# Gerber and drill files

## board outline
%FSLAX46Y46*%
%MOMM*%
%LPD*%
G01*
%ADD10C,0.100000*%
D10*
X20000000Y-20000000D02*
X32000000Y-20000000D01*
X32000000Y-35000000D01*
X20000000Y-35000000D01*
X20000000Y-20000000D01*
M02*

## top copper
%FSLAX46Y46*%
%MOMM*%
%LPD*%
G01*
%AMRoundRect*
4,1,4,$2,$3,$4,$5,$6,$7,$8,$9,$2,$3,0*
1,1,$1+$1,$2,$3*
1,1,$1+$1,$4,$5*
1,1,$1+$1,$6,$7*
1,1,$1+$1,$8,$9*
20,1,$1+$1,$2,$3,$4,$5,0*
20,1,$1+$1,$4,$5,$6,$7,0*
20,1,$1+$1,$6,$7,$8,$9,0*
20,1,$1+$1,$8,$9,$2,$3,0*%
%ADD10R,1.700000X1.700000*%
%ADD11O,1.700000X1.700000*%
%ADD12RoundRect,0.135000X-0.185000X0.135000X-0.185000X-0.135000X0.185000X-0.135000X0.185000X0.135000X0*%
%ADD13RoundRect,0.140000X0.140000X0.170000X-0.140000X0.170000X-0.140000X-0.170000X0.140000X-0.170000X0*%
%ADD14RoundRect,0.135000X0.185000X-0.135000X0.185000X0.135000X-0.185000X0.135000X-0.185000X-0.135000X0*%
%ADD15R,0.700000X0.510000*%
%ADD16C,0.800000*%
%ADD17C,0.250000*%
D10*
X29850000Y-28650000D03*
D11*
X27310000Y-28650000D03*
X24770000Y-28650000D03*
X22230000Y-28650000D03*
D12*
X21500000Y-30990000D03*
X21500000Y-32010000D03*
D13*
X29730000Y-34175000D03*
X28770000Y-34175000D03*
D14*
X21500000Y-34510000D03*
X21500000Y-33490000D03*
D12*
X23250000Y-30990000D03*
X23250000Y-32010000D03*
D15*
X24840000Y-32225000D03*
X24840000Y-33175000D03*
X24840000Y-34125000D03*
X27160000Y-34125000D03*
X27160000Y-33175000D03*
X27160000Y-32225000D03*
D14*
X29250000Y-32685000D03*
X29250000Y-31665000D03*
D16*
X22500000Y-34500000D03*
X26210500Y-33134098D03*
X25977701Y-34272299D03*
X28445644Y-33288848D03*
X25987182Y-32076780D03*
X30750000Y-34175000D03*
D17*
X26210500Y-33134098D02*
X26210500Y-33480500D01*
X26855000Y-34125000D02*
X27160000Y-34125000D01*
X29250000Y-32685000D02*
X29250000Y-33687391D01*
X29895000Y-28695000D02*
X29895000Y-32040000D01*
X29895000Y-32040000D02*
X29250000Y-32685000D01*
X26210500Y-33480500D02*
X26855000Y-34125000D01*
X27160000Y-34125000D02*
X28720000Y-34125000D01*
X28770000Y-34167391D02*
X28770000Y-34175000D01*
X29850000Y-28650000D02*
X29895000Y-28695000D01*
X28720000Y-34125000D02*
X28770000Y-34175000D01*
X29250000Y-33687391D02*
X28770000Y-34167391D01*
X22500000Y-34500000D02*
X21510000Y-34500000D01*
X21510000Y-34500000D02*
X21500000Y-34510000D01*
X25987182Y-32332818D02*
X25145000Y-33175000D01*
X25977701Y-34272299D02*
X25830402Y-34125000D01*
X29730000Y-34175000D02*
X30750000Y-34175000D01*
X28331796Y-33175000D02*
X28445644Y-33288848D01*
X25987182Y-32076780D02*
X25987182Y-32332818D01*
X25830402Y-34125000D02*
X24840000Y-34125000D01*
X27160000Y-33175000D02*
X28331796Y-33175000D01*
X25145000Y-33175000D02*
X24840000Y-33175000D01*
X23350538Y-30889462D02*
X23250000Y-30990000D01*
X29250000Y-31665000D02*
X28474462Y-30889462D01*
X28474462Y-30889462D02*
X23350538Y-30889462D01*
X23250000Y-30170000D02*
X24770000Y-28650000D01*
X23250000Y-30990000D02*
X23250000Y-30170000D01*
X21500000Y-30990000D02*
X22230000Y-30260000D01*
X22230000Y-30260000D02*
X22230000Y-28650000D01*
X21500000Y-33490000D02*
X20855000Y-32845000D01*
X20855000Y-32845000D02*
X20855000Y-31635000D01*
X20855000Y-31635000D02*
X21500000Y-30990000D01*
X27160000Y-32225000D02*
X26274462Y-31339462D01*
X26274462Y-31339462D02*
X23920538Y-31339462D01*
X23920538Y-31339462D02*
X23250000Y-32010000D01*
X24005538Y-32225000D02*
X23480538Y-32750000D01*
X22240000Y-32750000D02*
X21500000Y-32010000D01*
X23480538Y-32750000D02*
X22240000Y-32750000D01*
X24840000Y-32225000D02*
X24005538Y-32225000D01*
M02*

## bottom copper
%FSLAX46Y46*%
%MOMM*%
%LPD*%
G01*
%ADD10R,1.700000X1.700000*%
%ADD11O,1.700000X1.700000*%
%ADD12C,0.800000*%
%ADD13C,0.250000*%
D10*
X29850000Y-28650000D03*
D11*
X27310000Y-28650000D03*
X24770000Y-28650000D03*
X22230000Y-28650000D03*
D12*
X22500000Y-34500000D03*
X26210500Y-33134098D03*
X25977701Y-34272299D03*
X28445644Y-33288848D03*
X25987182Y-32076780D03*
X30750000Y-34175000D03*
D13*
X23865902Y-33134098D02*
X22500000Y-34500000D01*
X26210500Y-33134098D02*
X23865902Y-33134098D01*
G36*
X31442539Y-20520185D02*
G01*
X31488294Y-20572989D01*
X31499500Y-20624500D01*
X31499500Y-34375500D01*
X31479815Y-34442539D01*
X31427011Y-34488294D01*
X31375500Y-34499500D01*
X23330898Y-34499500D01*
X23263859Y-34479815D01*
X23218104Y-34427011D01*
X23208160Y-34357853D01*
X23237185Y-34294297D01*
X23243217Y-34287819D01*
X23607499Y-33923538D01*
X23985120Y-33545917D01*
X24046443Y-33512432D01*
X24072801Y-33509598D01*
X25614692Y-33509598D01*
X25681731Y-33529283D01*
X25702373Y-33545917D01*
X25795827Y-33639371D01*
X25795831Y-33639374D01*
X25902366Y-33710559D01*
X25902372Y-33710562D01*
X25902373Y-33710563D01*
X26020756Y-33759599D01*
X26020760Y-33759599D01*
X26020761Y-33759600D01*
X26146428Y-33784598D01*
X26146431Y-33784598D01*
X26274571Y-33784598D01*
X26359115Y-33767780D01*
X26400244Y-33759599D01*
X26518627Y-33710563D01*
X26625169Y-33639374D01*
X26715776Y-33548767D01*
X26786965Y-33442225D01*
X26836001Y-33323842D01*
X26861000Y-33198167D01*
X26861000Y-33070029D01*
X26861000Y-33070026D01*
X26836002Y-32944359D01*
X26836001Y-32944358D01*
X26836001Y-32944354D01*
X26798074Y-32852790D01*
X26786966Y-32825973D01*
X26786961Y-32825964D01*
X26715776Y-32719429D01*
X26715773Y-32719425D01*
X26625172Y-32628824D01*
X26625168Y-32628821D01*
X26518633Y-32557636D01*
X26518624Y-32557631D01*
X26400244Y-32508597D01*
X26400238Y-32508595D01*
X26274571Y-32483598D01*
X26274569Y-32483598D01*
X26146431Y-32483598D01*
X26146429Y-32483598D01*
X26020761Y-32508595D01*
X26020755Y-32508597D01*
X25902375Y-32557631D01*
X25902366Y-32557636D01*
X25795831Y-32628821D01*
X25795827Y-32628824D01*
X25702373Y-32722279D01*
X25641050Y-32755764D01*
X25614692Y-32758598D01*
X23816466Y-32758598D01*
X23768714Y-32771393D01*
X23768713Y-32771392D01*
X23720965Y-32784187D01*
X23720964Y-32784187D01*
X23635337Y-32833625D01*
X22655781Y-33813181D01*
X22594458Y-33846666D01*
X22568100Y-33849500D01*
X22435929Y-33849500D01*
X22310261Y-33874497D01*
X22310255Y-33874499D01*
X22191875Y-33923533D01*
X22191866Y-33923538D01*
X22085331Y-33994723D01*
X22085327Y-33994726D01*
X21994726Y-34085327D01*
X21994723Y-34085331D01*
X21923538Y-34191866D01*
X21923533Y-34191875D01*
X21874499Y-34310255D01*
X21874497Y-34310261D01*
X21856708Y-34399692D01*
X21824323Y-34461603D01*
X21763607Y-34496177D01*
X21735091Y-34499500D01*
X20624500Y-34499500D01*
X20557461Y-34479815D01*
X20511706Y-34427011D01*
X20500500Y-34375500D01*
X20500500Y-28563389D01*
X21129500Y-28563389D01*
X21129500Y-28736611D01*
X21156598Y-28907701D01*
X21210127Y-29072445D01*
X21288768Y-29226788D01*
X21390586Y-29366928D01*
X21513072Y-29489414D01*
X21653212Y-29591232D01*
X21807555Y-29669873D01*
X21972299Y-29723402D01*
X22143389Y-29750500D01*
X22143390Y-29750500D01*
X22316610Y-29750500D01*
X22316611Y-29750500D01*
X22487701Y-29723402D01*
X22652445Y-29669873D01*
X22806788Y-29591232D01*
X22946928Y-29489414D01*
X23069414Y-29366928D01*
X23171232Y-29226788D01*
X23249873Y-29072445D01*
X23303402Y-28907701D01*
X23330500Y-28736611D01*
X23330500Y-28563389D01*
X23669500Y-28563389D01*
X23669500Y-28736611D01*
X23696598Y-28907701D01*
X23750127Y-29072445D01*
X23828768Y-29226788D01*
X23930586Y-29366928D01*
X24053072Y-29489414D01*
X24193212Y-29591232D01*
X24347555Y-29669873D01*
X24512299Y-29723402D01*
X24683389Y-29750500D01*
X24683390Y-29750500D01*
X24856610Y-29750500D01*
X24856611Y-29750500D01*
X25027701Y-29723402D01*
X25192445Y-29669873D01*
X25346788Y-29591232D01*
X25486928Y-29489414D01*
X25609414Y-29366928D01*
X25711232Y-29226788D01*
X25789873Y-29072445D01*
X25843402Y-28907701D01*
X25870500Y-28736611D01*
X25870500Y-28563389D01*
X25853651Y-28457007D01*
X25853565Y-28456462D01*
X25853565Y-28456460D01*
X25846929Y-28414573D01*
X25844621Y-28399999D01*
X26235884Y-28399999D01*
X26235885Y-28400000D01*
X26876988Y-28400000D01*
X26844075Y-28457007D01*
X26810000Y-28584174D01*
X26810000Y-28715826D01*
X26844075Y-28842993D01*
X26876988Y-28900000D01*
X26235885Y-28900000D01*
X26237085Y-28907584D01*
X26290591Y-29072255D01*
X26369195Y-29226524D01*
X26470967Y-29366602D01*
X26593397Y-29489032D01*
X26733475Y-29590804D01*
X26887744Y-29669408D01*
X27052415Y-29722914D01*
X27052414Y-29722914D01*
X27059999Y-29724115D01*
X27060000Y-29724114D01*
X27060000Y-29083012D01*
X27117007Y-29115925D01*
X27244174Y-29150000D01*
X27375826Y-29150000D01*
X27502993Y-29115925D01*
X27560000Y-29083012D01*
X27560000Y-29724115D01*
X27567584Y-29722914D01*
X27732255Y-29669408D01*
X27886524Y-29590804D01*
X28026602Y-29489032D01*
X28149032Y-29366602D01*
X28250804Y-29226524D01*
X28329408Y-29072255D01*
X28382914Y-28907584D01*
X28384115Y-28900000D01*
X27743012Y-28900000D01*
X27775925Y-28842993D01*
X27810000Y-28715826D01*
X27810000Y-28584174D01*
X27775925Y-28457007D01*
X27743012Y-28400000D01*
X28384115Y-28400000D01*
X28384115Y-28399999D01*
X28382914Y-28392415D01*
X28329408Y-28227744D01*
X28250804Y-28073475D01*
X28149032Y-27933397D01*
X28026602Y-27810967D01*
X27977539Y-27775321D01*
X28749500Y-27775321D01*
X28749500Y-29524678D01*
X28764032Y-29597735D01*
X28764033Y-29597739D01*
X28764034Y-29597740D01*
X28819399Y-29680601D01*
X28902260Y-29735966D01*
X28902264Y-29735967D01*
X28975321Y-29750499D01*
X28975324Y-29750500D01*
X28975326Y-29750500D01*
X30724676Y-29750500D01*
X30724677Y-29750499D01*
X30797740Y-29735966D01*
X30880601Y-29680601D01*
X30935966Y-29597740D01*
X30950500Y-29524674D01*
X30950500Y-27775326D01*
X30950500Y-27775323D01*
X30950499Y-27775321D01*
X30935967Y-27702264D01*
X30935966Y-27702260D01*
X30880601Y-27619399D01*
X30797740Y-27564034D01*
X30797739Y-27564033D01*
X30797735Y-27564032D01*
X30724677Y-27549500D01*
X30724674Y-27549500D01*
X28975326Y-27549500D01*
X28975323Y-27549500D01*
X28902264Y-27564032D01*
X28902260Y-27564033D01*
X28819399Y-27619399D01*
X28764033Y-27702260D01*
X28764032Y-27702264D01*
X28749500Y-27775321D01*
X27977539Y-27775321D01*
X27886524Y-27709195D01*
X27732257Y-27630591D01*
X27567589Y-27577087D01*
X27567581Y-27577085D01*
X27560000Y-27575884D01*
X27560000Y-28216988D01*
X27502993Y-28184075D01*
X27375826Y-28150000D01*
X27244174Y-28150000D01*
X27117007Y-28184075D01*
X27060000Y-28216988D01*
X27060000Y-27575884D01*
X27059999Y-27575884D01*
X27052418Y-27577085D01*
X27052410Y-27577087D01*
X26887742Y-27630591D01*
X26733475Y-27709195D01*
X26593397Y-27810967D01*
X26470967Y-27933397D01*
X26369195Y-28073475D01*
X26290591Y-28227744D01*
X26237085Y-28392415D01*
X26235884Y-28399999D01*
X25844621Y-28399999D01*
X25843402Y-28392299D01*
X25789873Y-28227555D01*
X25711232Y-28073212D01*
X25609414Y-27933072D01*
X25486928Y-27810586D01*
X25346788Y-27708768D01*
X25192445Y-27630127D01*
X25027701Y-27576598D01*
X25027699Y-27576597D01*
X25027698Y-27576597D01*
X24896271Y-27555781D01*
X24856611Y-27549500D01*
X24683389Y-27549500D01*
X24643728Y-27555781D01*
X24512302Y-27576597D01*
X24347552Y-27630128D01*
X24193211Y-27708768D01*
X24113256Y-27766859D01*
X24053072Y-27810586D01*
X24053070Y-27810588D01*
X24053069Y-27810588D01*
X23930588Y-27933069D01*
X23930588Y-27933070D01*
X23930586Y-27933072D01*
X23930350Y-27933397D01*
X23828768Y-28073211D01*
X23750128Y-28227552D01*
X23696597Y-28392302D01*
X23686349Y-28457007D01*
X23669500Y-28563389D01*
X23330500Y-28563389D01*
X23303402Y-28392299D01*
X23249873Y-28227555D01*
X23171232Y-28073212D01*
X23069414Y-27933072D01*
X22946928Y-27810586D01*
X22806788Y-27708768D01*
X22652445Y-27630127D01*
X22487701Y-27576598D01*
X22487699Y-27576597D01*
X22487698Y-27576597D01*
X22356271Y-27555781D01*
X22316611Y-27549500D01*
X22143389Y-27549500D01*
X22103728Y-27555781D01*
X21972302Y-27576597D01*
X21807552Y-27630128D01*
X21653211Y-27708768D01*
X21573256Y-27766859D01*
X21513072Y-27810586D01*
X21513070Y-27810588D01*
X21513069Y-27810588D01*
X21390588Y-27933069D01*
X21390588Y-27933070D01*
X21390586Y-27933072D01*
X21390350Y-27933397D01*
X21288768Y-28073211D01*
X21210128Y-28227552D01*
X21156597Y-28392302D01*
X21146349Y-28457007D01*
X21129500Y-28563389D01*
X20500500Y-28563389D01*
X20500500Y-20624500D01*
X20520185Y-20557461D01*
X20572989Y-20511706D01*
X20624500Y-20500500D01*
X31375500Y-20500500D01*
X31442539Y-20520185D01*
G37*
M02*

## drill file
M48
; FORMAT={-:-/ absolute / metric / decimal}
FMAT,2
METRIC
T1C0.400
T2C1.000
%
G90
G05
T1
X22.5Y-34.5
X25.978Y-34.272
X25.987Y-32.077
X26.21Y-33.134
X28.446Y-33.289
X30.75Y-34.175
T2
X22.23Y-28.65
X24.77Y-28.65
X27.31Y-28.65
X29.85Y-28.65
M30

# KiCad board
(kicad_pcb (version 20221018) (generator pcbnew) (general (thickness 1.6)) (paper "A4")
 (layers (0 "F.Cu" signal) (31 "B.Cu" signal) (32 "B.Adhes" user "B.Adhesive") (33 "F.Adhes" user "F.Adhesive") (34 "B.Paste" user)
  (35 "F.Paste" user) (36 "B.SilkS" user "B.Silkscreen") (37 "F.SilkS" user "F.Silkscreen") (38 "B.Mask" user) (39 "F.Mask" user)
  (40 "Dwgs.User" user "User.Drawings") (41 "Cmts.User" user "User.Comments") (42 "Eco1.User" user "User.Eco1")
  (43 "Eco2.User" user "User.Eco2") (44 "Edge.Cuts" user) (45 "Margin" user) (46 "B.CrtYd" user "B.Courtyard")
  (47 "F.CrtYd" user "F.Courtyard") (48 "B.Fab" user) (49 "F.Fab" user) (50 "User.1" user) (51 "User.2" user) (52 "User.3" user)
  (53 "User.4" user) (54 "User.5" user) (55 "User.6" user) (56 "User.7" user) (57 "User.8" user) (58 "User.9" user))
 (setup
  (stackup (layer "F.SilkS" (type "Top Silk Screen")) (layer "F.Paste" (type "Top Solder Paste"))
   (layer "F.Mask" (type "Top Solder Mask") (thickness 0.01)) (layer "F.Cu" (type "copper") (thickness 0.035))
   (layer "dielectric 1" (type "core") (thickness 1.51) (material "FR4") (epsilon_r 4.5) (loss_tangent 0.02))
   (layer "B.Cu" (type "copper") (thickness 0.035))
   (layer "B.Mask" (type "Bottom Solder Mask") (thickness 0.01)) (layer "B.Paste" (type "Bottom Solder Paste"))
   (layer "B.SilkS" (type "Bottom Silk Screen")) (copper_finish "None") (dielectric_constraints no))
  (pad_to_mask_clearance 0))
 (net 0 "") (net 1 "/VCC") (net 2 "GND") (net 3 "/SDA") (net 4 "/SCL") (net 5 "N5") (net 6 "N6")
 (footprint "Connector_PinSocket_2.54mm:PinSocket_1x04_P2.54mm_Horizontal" (layer "F.Cu") (at 29.85 28.65 -90)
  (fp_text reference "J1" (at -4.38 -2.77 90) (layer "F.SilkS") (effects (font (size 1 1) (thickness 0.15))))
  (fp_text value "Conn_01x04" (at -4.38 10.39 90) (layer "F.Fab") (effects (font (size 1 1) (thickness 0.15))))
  (pad "1" thru_hole rect (at 0 0 270) (size 1.7 1.7) (drill 1) (layers "*.Cu" "*.Mask") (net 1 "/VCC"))
  (pad "2" thru_hole oval (at 0 2.54 270) (size 1.7 1.7) (drill 1) (layers "*.Cu" "*.Mask") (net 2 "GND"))
  (pad "3" thru_hole oval (at 0 5.08 270) (size 1.7 1.7) (drill 1) (layers "*.Cu" "*.Mask") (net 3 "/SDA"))
  (pad "4" thru_hole oval (at 0 7.62 270) (size 1.7 1.7) (drill 1) (layers "*.Cu" "*.Mask") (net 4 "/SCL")))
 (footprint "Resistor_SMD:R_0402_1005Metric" (layer "F.Cu") (at 21.5 31.5 -90)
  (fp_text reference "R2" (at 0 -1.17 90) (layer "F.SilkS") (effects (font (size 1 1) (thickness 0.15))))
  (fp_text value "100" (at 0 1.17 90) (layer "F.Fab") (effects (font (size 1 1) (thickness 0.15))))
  (pad "1" smd roundrect (at -0.51 0 270) (size 0.54 0.64) (layers "F.Cu" "F.Paste" "F.Mask") (roundrect_rratio 0.25) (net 4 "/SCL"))
  (pad "2" smd roundrect (at 0.51 0 270) (size 0.54 0.64) (layers "F.Cu" "F.Paste" "F.Mask") (roundrect_rratio 0.25) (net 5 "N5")))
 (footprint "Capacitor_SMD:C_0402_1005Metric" (layer "F.Cu") (at 29.25 34.175 180)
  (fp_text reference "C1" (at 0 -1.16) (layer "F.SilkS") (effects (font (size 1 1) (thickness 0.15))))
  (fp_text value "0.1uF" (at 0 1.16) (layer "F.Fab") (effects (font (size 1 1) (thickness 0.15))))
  (pad "1" smd roundrect (at -0.48 0 180) (size 0.56 0.62) (layers "F.Cu" "F.Paste" "F.Mask") (roundrect_rratio 0.25) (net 2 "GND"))
  (pad "2" smd roundrect (at 0.48 0 180) (size 0.56 0.62) (layers "F.Cu" "F.Paste" "F.Mask") (roundrect_rratio 0.25) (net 1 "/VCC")))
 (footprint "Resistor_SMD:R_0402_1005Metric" (layer "F.Cu") (at 21.5 34 90)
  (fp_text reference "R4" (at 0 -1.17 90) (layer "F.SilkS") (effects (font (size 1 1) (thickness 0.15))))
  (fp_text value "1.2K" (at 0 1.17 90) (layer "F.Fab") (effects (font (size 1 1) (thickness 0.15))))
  (pad "1" smd roundrect (at -0.51 0 90) (size 0.54 0.64) (layers "F.Cu" "F.Paste" "F.Mask") (roundrect_rratio 0.25) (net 1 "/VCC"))
  (pad "2" smd roundrect (at 0.51 0 90) (size 0.54 0.64) (layers "F.Cu" "F.Paste" "F.Mask") (roundrect_rratio 0.25) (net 4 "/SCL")))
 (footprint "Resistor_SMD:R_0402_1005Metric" (layer "F.Cu") (at 23.25 31.5 -90)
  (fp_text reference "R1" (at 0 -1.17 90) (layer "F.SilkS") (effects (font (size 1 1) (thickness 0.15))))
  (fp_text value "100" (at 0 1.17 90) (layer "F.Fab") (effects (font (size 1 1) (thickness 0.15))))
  (pad "1" smd roundrect (at -0.51 0 270) (size 0.54 0.64) (layers "F.Cu" "F.Paste" "F.Mask") (roundrect_rratio 0.25) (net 3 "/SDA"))
  (pad "2" smd roundrect (at 0.51 0 270) (size 0.54 0.64) (layers "F.Cu" "F.Paste" "F.Mask") (roundrect_rratio 0.25) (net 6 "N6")))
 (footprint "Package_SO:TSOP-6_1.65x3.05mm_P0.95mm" (layer "F.Cu") (at 26 33.175)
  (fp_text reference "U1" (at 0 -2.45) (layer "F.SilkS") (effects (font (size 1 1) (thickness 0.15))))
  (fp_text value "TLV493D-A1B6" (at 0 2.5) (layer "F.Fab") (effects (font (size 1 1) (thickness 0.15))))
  (pad "1" smd rect (at -1.16 -0.95) (size 0.7 0.51) (layers "F.Cu" "F.Paste" "F.Mask") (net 5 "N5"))
  (pad "2" smd rect (at -1.16 0) (size 0.7 0.51) (layers "F.Cu" "F.Paste" "F.Mask") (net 2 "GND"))
  (pad "3" smd rect (at -1.16 0.95) (size 0.7 0.51) (layers "F.Cu" "F.Paste" "F.Mask") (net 2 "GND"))
  (pad "4" smd rect (at 1.16 0.95) (size 0.7 0.51) (layers "F.Cu" "F.Paste" "F.Mask") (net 1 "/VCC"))
  (pad "5" smd rect (at 1.16 0) (size 0.7 0.51) (layers "F.Cu" "F.Paste" "F.Mask") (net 2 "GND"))
  (pad "6" smd rect (at 1.16 -0.95) (size 0.7 0.51) (layers "F.Cu" "F.Paste" "F.Mask") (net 6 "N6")))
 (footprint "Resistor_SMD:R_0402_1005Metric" (layer "F.Cu") (at 29.25 32.175 90)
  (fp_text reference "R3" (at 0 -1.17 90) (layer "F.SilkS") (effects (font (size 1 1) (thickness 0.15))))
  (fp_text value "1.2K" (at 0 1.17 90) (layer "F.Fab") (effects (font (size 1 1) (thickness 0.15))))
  (pad "1" smd roundrect (at -0.51 0 90) (size 0.54 0.64) (layers "F.Cu" "F.Paste" "F.Mask") (roundrect_rratio 0.25) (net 1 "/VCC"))
  (pad "2" smd roundrect (at 0.51 0 90) (size 0.54 0.64) (layers "F.Cu" "F.Paste" "F.Mask") (roundrect_rratio 0.25) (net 3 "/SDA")))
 (gr_rect (start 20 20) (end 32 35) (stroke (width 0.1) (type default)) (fill none) (layer "Edge.Cuts"))
 (segment (start 26.2105 33.134098) (end 26.2105 33.4805) (width 0.25) (layer "F.Cu") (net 1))
 (segment (start 26.855 34.125) (end 27.16 34.125) (width 0.25) (layer "F.Cu") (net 1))
 (segment (start 29.25 32.685) (end 29.25 33.687391) (width 0.25) (layer "F.Cu") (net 1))
 (segment (start 29.895 28.695) (end 29.895 32.04) (width 0.25) (layer "F.Cu") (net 1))
 (segment (start 29.895 32.04) (end 29.25 32.685) (width 0.25) (layer "F.Cu") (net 1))
 (segment (start 26.2105 33.4805) (end 26.855 34.125) (width 0.25) (layer "F.Cu") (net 1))
 (segment (start 27.16 34.125) (end 28.72 34.125) (width 0.25) (layer "F.Cu") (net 1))
 (segment (start 28.77 34.167391) (end 28.77 34.175) (width 0.25) (layer "F.Cu") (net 1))
 (segment (start 29.85 28.65) (end 29.895 28.695) (width 0.25) (layer "F.Cu") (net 1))
 (segment (start 28.72 34.125) (end 28.77 34.175) (width 0.25) (layer "F.Cu") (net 1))
 (segment (start 29.25 33.687391) (end 28.77 34.167391) (width 0.25) (layer "F.Cu") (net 1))
 (segment (start 22.5 34.5) (end 21.51 34.5) (width 0.25) (layer "F.Cu") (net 1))
 (segment (start 21.51 34.5) (end 21.5 34.51) (width 0.25) (layer "F.Cu") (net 1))
 (via (at 22.5 34.5) (size 0.8) (drill 0.4) (layers "F.Cu" "B.Cu") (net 1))
 (via (at 26.2105 33.134098) (size 0.8) (drill 0.4) (layers "F.Cu" "B.Cu") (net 1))
 (segment (start 23.865902 33.134098) (end 22.5 34.5) (width 0.25) (layer "B.Cu") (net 1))
 (segment (start 26.2105 33.134098) (end 23.865902 33.134098) (width 0.25) (layer "B.Cu") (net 1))
 (segment (start 25.987182 32.332818) (end 25.145 33.175) (width 0.25) (layer "F.Cu") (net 2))
 (segment (start 25.977701 34.272299) (end 25.830402 34.125) (width 0.25) (layer "F.Cu") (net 2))
 (segment (start 29.73 34.175) (end 30.75 34.175) (width 0.25) (layer "F.Cu") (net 2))
 (segment (start 28.331796 33.175) (end 28.445644 33.288848) (width 0.25) (layer "F.Cu") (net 2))
 (segment (start 25.987182 32.07678) (end 25.987182 32.332818) (width 0.25) (layer "F.Cu") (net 2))
 (segment (start 25.830402 34.125) (end 24.84 34.125) (width 0.25) (layer "F.Cu") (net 2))
 (segment (start 27.16 33.175) (end 28.331796 33.175) (width 0.25) (layer "F.Cu") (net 2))
 (segment (start 25.145 33.175) (end 24.84 33.175) (width 0.25) (layer "F.Cu") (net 2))
 (via (at 25.977701 34.272299) (size 0.8) (drill 0.4) (layers "F.Cu" "B.Cu") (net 2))
 (via (at 28.445644 33.288848) (size 0.8) (drill 0.4) (layers "F.Cu" "B.Cu") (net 2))
 (via (at 25.987182 32.07678) (size 0.8) (drill 0.4) (layers "F.Cu" "B.Cu") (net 2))
 (via (at 30.75 34.175) (size 0.8) (drill 0.4) (layers "F.Cu" "B.Cu") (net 2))
 (segment (start 23.350538 30.889462) (end 23.25 30.99) (width 0.25) (layer "F.Cu") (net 3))
 (segment (start 29.25 31.665) (end 28.474462 30.889462) (width 0.25) (layer "F.Cu") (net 3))
 (segment (start 28.474462 30.889462) (end 23.350538 30.889462) (width 0.25) (layer "F.Cu") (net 3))
 (segment (start 23.25 30.17) (end 24.77 28.65) (width 0.25) (layer "F.Cu") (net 3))
 (segment (start 23.25 30.99) (end 23.25 30.17) (width 0.25) (layer "F.Cu") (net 3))
 (segment (start 21.5 30.99) (end 22.23 30.26) (width 0.25) (layer "F.Cu") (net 4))
 (segment (start 22.23 30.26) (end 22.23 28.65) (width 0.25) (layer "F.Cu") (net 4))
 (segment (start 21.5 33.49) (end 20.855 32.845) (width 0.25) (layer "F.Cu") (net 4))
 (segment (start 20.855 32.845) (end 20.855 31.635) (width 0.25) (layer "F.Cu") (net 4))
 (segment (start 20.855 31.635) (end 21.5 30.99) (width 0.25) (layer "F.Cu") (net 4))
 (segment (start 27.16 32.225) (end 26.274462 31.339462) (width 0.25) (layer "F.Cu") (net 6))
 (segment (start 26.274462 31.339462) (end 23.920538 31.339462) (width 0.25) (layer "F.Cu") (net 6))
 (segment (start 23.920538 31.339462) (end 23.25 32.01) (width 0.25) (layer "F.Cu") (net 6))
 (segment (start 24.005538 32.225) (end 23.480538 32.75) (width 0.25) (layer "F.Cu") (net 5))
 (segment (start 22.24 32.75) (end 21.5 32.01) (width 0.25) (layer "F.Cu") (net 5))
 (segment (start 23.480538 32.75) (end 22.24 32.75) (width 0.25) (layer "F.Cu") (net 5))
 (segment (start 24.84 32.225) (end 24.005538 32.225) (width 0.25) (layer "F.Cu") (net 5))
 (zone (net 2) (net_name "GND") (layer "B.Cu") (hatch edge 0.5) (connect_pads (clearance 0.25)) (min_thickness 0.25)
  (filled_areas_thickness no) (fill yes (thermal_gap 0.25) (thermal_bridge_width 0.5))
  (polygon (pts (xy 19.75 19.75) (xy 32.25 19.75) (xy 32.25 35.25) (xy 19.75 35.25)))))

